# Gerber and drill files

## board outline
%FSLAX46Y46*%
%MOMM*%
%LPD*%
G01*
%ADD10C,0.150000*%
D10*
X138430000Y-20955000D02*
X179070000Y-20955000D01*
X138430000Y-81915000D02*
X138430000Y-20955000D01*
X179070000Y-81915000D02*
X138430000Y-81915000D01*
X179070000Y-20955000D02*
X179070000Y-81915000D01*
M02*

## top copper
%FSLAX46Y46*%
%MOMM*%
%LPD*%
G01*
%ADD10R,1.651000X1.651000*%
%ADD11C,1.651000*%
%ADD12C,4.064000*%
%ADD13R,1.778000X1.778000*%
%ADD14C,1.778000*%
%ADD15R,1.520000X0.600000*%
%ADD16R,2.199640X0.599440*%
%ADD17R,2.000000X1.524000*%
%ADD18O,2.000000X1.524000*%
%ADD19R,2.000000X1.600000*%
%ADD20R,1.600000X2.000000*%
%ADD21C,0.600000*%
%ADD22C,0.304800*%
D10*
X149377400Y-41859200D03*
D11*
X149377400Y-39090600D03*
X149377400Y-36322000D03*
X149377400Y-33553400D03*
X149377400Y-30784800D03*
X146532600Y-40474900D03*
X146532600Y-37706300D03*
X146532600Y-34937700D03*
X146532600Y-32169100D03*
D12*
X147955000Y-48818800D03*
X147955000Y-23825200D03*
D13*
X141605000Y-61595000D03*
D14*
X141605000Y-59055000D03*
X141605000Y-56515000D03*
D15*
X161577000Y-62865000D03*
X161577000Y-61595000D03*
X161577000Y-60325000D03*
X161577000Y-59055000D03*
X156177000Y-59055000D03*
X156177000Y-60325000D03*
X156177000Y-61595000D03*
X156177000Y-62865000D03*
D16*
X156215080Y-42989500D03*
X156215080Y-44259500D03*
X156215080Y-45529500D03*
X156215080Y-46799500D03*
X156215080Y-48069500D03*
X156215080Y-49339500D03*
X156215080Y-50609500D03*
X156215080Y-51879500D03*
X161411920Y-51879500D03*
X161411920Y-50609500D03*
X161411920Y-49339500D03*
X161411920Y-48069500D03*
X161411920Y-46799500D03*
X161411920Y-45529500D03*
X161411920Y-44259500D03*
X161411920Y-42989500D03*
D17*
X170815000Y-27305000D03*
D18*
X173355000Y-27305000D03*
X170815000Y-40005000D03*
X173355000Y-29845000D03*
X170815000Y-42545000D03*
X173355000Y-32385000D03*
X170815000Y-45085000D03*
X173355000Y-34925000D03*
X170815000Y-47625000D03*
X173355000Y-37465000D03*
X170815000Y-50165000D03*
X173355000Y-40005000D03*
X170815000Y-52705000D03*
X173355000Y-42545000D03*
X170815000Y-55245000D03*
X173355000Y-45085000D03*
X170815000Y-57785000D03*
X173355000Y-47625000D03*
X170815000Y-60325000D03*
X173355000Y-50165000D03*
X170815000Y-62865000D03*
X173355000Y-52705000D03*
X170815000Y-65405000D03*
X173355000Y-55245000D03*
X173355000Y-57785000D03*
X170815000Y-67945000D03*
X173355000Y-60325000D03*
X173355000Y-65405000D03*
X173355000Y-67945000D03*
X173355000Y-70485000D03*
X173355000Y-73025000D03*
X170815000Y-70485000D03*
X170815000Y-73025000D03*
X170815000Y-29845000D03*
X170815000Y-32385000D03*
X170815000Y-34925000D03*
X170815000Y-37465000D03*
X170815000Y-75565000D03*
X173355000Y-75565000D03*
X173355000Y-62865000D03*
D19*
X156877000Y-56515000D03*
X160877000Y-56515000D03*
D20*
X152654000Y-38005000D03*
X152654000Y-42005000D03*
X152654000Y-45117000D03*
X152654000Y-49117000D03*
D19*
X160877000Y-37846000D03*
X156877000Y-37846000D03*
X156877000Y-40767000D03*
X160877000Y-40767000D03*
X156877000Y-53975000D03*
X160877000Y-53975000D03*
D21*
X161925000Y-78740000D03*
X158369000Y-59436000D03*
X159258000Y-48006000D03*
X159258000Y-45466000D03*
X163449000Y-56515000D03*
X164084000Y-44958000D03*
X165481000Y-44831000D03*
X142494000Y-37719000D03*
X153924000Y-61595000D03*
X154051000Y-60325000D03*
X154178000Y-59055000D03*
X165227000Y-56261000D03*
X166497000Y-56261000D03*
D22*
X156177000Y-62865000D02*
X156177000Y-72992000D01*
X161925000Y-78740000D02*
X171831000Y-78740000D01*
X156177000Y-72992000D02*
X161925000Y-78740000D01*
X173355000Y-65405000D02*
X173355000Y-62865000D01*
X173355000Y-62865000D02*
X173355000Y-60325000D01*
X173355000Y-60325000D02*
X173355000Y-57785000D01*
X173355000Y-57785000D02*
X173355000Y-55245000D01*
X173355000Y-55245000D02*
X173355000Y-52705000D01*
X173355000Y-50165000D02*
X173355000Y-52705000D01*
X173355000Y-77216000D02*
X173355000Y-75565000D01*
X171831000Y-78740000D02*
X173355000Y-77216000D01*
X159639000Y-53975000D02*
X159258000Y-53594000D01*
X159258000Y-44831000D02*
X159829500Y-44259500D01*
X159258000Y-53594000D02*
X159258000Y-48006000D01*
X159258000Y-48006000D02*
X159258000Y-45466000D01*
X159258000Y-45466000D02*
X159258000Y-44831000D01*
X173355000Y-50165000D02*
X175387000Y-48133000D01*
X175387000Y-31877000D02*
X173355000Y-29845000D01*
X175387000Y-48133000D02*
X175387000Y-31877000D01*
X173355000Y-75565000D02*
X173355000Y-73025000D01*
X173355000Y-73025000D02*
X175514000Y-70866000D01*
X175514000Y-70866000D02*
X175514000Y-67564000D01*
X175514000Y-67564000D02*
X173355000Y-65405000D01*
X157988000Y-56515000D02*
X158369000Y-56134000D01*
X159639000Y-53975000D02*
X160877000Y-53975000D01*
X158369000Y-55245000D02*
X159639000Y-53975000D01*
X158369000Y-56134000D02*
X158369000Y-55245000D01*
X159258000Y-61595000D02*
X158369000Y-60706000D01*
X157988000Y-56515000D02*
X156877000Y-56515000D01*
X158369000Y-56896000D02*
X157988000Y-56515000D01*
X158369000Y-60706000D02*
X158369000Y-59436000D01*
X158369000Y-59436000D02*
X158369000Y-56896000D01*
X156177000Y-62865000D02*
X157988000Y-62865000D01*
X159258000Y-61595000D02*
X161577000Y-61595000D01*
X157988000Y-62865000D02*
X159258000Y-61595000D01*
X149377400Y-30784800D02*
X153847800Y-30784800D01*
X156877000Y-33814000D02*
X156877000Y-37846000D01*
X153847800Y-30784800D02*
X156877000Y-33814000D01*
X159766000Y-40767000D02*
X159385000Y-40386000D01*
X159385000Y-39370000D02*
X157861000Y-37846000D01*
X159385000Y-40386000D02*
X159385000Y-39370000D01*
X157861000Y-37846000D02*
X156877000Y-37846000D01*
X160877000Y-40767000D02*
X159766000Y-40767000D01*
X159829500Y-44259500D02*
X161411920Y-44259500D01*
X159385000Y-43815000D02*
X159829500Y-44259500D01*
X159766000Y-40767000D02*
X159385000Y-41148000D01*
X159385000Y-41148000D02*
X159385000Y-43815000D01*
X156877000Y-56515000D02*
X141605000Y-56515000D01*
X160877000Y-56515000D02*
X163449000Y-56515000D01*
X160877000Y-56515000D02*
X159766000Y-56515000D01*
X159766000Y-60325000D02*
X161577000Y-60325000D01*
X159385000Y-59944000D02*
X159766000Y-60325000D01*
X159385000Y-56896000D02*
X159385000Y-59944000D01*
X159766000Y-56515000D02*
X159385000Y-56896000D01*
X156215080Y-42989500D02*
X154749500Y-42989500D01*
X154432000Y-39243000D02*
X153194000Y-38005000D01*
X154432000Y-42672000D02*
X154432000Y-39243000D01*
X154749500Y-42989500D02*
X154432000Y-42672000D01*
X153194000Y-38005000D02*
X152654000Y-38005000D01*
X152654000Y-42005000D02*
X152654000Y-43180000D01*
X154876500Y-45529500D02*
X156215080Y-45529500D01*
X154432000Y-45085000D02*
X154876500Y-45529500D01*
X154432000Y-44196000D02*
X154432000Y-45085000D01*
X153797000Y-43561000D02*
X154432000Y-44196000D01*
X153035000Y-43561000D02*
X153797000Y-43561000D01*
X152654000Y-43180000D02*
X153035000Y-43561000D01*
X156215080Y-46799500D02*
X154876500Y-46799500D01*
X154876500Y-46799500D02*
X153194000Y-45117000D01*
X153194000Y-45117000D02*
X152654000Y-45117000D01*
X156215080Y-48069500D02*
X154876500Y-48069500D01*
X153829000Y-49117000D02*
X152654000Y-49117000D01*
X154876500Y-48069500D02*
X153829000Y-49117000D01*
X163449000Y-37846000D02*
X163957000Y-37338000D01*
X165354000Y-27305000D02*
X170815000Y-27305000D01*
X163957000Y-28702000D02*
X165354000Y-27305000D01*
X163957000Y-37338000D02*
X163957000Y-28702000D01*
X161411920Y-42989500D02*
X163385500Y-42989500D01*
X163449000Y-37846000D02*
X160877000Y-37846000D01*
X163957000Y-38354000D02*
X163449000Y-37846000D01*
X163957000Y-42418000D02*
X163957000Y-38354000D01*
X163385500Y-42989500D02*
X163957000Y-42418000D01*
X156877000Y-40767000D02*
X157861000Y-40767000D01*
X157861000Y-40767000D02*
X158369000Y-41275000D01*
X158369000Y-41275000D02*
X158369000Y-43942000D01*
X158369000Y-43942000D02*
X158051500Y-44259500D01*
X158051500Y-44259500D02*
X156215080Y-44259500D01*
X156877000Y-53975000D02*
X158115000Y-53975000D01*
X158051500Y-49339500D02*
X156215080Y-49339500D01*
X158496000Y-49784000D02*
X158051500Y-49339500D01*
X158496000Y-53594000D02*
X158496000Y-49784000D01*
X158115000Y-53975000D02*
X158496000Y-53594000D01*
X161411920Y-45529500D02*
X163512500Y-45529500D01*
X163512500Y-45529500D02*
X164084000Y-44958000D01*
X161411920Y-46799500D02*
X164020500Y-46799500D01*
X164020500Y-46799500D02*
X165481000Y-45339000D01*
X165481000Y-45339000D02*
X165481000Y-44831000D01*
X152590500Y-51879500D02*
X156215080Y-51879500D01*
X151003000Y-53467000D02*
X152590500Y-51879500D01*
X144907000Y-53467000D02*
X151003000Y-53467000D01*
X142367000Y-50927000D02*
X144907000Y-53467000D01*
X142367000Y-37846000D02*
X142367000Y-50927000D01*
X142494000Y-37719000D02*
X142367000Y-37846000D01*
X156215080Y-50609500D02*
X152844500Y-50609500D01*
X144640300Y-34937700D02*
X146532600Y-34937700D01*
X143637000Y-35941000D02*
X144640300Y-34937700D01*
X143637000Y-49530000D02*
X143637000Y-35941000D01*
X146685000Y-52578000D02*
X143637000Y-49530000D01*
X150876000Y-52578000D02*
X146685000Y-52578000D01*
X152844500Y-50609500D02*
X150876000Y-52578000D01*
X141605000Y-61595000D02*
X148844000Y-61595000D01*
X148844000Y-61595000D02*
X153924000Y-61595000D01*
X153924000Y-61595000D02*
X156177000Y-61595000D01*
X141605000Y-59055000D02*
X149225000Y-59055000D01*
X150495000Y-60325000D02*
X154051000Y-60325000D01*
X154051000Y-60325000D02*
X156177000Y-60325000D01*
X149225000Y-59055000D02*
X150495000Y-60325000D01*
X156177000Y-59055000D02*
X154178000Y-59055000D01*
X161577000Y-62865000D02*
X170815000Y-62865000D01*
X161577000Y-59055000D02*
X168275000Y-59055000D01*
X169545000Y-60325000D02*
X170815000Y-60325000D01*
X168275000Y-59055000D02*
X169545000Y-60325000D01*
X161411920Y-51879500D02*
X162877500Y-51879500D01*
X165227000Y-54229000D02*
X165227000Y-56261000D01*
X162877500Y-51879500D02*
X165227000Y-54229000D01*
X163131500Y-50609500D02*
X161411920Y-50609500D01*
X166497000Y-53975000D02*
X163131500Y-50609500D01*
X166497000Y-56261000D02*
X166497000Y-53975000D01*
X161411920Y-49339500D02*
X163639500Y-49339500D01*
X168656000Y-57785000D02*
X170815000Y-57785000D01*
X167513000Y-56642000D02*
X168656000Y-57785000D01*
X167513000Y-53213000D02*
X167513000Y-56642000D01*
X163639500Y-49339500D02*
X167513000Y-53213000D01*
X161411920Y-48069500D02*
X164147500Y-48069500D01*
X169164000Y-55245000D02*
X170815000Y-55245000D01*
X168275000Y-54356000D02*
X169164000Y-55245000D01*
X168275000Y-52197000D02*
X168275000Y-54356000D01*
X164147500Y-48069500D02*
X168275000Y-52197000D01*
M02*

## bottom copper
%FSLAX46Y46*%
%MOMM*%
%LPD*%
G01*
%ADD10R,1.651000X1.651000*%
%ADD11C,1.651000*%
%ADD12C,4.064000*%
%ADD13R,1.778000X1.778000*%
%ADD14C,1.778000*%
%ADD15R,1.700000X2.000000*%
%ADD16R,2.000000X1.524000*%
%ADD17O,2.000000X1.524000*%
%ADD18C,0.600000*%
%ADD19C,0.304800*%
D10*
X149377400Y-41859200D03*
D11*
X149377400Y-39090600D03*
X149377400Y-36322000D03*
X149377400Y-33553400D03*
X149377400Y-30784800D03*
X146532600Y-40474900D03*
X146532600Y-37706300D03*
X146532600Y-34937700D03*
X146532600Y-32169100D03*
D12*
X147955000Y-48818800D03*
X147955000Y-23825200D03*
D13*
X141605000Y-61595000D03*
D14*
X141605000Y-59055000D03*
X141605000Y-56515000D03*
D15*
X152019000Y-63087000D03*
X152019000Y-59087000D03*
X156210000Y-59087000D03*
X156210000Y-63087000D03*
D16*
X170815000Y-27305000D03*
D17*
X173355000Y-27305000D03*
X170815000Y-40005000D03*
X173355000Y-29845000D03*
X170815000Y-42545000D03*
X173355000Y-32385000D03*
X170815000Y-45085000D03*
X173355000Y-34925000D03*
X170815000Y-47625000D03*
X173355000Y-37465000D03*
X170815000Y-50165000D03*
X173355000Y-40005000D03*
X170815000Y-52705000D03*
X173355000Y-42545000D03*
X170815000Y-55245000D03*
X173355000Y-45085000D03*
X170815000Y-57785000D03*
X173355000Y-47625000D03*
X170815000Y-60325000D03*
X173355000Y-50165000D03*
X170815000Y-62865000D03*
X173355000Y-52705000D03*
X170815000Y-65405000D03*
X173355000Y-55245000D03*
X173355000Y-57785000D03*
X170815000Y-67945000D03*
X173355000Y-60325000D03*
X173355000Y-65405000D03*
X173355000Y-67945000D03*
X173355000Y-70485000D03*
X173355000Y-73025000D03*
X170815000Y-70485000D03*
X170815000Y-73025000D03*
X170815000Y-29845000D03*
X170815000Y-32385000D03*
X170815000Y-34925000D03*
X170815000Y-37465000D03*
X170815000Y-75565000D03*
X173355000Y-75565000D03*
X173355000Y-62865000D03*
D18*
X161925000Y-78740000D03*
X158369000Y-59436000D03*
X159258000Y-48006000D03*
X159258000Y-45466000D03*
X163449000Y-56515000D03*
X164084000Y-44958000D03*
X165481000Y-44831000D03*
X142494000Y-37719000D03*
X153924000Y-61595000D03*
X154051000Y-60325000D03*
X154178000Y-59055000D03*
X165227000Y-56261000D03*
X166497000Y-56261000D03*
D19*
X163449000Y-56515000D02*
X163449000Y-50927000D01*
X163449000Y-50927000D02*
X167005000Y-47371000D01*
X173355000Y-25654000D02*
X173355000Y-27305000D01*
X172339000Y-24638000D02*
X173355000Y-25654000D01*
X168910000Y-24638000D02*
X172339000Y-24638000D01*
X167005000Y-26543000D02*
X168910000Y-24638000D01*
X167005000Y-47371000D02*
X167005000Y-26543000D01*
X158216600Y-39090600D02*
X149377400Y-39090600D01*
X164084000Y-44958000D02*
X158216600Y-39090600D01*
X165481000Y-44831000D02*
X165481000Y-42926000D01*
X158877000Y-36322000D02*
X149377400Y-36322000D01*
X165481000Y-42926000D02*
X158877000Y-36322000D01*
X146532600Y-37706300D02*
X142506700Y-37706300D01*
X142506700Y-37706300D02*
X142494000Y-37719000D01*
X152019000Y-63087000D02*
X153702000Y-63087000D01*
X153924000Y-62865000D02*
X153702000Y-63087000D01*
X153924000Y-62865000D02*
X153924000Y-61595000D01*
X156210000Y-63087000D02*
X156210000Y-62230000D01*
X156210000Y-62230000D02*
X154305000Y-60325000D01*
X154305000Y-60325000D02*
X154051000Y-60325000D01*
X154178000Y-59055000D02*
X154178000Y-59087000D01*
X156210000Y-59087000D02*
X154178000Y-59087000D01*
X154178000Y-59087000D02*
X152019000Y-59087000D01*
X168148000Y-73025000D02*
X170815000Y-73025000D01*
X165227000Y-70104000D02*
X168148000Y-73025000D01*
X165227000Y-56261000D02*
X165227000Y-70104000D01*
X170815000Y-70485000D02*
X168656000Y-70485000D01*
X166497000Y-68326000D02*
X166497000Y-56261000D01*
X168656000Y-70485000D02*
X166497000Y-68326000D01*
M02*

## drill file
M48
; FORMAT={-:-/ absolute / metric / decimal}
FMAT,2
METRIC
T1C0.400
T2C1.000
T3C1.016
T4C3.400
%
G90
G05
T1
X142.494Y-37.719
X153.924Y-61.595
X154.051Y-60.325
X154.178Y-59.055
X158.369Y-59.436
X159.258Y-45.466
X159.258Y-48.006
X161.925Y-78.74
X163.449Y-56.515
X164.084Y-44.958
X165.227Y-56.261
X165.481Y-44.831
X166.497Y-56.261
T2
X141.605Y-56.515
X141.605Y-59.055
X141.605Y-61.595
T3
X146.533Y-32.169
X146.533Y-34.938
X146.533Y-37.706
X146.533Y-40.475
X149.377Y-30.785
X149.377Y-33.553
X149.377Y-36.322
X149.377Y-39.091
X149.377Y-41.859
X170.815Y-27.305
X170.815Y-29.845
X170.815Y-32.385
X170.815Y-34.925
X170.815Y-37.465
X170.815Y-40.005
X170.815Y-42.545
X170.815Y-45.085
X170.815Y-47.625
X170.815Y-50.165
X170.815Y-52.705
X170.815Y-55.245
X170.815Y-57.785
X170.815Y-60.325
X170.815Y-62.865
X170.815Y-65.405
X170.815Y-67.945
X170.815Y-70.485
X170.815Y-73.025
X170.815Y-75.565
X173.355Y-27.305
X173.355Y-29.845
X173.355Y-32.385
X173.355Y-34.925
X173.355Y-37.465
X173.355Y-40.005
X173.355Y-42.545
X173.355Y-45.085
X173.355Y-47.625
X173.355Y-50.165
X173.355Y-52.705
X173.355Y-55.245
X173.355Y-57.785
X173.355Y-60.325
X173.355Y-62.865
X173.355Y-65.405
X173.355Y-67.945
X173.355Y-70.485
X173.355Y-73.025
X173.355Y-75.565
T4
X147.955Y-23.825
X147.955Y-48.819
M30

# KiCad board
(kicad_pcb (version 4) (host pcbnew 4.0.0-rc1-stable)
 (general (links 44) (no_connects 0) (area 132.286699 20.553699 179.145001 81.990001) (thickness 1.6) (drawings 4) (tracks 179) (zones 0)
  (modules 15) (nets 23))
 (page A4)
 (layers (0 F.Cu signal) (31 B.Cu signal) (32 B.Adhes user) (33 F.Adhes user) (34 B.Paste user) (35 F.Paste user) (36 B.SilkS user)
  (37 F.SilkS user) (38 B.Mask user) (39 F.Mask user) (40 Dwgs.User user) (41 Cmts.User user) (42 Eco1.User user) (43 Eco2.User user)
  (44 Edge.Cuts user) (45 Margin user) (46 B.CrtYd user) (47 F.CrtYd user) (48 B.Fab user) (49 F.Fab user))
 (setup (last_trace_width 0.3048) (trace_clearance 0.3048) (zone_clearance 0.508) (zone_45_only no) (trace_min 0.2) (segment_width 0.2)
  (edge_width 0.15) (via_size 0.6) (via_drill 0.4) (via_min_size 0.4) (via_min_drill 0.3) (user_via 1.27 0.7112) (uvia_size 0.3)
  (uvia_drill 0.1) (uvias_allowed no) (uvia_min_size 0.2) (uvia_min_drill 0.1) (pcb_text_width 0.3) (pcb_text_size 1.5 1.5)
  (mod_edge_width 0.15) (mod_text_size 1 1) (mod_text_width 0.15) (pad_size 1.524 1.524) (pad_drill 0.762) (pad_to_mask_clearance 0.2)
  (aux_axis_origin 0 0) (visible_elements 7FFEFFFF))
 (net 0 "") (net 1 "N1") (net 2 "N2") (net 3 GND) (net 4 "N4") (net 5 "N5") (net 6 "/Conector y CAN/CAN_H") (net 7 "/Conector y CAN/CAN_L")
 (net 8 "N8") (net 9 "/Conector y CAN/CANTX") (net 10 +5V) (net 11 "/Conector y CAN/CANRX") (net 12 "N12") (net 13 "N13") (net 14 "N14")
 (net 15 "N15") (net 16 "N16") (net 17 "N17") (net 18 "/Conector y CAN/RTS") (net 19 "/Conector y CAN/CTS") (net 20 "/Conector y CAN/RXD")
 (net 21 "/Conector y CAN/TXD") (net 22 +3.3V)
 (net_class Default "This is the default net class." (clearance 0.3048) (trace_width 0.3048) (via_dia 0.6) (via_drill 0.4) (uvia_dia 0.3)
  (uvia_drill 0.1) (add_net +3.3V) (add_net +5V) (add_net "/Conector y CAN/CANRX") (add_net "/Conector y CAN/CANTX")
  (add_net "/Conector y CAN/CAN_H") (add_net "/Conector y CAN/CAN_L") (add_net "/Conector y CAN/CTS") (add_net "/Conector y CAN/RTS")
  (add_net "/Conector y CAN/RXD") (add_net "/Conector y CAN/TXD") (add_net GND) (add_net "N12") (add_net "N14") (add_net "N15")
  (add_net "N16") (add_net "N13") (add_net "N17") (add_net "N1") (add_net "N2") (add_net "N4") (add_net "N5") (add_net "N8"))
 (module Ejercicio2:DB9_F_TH (layer F.Cu) (at 147.955 36.322 90)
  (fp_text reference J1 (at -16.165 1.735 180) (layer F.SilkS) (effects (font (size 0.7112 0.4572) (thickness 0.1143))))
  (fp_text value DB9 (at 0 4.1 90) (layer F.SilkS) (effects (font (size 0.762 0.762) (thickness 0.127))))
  (pad 1 thru_hole rect (at -5.5372 1.4224 90) (size 1.651 1.651) (drill 1.016) (layers *.Cu *.Mask))
  (pad 2 thru_hole circle (at -2.7686 1.4224 90) (size 1.651 1.651) (drill 1.016) (layers *.Cu *.Mask) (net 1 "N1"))
  (pad 3 thru_hole circle (at 0 1.4224 90) (size 1.651 1.651) (drill 1.016) (layers *.Cu *.Mask) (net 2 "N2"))
  (pad 4 thru_hole circle (at 2.7686 1.4224 90) (size 1.651 1.651) (drill 1.016) (layers *.Cu *.Mask))
  (pad 5 thru_hole circle (at 5.5372 1.4224 90) (size 1.651 1.651) (drill 1.016) (layers *.Cu *.Mask) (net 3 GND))
  (pad 6 thru_hole circle (at -4.1529 -1.4224 90) (size 1.651 1.651) (drill 1.016) (layers *.Cu *.Mask))
  (pad 7 thru_hole circle (at -1.3843 -1.4224 90) (size 1.651 1.651) (drill 1.016) (layers *.Cu *.Mask) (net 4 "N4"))
  (pad 8 thru_hole circle (at 1.3843 -1.4224 90) (size 1.651 1.651) (drill 1.016) (layers *.Cu *.Mask) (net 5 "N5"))
  (pad 9 thru_hole circle (at 4.1529 -1.4224 90) (size 1.651 1.651) (drill 1.016) (layers *.Cu *.Mask))
  (pad 10 thru_hole circle (at -12.4968 0 90) (size 4.064 4.064) (drill 3.4) (layers *.Cu *.Mask))
  (pad 11 thru_hole circle (at 12.4968 0 90) (size 4.064 4.064) (drill 3.4) (layers *.Cu *.Mask)))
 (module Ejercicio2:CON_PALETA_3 (layer F.Cu) (at 141.605 59.055 90)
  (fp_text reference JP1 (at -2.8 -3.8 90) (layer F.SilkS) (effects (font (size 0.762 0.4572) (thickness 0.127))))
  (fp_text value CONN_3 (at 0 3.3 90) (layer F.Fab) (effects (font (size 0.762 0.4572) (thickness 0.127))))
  (pad 1 thru_hole rect (at -2.54 0 90) (size 1.778 1.778) (drill 1) (layers *.Cu *.Mask) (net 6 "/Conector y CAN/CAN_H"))
  (pad 2 thru_hole circle (at 0 0 90) (size 1.778 1.778) (drill 1) (layers *.Cu *.Mask) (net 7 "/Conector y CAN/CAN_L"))
  (pad 3 thru_hole circle (at 2.54 0 90) (size 1.778 1.778) (drill 1) (layers *.Cu *.Mask) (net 3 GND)))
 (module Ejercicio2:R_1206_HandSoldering (layer B.Cu) (at 152.019 61.087 90)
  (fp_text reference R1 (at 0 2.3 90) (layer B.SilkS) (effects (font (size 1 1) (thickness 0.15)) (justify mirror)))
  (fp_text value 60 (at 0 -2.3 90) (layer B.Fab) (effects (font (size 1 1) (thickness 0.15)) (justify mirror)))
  (pad 1 smd rect (at -2 0 90) (size 2 1.7) (layers B.Cu B.Paste B.Mask) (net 6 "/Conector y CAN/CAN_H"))
  (pad 2 smd rect (at 2 0 90) (size 2 1.7) (layers B.Cu B.Paste B.Mask) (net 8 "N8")))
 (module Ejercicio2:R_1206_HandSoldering (layer B.Cu) (at 156.21 61.087 270)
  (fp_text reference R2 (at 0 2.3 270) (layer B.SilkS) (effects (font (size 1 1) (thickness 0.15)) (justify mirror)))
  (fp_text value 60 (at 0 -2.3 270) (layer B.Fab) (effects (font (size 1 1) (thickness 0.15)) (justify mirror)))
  (pad 1 smd rect (at -2 0 270) (size 2 1.7) (layers B.Cu B.Paste B.Mask) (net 8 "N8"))
  (pad 2 smd rect (at 2 0 270) (size 2 1.7) (layers B.Cu B.Paste B.Mask) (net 7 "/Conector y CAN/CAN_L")))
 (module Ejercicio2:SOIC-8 (layer F.Cu) (at 158.877 60.96 180)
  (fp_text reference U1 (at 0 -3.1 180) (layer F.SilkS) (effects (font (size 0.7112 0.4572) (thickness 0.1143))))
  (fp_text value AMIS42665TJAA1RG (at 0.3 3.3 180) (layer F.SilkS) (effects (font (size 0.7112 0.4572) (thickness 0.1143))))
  (pad 1 smd rect (at -2.7 -1.905 90) (size 0.6 1.52) (layers F.Cu F.Paste F.Mask) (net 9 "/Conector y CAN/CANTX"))
  (pad 2 smd rect (at -2.7 -0.635 90) (size 0.6 1.52) (layers F.Cu F.Paste F.Mask) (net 3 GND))
  (pad 3 smd rect (at -2.7 0.635 90) (size 0.6 1.52) (layers F.Cu F.Paste F.Mask) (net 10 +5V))
  (pad 4 smd rect (at -2.7 1.905 90) (size 0.6 1.52) (layers F.Cu F.Paste F.Mask) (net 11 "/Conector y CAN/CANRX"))
  (pad 5 smd rect (at 2.7 1.905 90) (size 0.6 1.52) (layers F.Cu F.Paste F.Mask) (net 8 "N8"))
  (pad 6 smd rect (at 2.7 0.635 90) (size 0.6 1.52) (layers F.Cu F.Paste F.Mask) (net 7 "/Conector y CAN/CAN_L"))
  (pad 7 smd rect (at 2.7 -0.635 90) (size 0.6 1.52) (layers F.Cu F.Paste F.Mask) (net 6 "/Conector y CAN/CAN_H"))
  (pad 8 smd rect (at 2.7 -1.905 90) (size 0.6 1.52) (layers F.Cu F.Paste F.Mask) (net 3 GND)))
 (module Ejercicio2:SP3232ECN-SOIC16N (layer F.Cu) (at 158.8135 47.4345 270)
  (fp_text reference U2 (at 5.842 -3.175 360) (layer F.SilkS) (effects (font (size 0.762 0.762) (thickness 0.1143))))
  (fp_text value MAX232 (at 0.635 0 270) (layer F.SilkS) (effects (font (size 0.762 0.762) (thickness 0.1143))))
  (pad 1 smd rect (at -4.445 2.59842 270) (size 0.59944 2.19964) (layers F.Cu F.Paste F.Mask) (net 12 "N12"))
  (pad 2 smd rect (at -3.175 2.59842 270) (size 0.59944 2.19964) (layers F.Cu F.Paste F.Mask) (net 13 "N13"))
  (pad 3 smd rect (at -1.905 2.59842 270) (size 0.59944 2.19964) (layers F.Cu F.Paste F.Mask) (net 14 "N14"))
  (pad 4 smd rect (at -0.635 2.59842 270) (size 0.59944 2.19964) (layers F.Cu F.Paste F.Mask) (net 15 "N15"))
  (pad 5 smd rect (at 0.635 2.59842 270) (size 0.59944 2.19964) (layers F.Cu F.Paste F.Mask) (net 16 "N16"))
  (pad 6 smd rect (at 1.905 2.59842 270) (size 0.59944 2.19964) (layers F.Cu F.Paste F.Mask) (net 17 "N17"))
  (pad 7 smd rect (at 3.175 2.59842 270) (size 0.59944 2.19964) (layers F.Cu F.Paste F.Mask) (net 5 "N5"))
  (pad 8 smd rect (at 4.445 2.59842 270) (size 0.59944 2.19964) (layers F.Cu F.Paste F.Mask) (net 4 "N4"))
  (pad 9 smd rect (at 4.445 -2.59842 270) (size 0.59944 2.19964) (layers F.Cu F.Paste F.Mask) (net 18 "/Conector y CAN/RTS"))
  (pad 10 smd rect (at 3.175 -2.59842 270) (size 0.59944 2.19964) (layers F.Cu F.Paste F.Mask) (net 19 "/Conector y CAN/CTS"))
  (pad 11 smd rect (at 1.905 -2.59842 270) (size 0.59944 2.19964) (layers F.Cu F.Paste F.Mask) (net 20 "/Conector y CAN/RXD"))
  (pad 12 smd rect (at 0.635 -2.59842 270) (size 0.59944 2.19964) (layers F.Cu F.Paste F.Mask) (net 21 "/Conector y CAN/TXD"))
  (pad 13 smd rect (at -0.635 -2.59842 270) (size 0.59944 2.19964) (layers F.Cu F.Paste F.Mask) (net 2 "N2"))
  (pad 14 smd rect (at -1.905 -2.59842 270) (size 0.59944 2.19964) (layers F.Cu F.Paste F.Mask) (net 1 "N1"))
  (pad 15 smd rect (at -3.175 -2.59842 270) (size 0.59944 2.19964) (layers F.Cu F.Paste F.Mask) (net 3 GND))
  (pad 16 smd rect (at -4.445 -2.59842 270) (size 0.59944 2.19964) (layers F.Cu F.Paste F.Mask) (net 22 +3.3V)))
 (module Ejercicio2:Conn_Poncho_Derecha (layer F.Cu) (at 170.815 27.305)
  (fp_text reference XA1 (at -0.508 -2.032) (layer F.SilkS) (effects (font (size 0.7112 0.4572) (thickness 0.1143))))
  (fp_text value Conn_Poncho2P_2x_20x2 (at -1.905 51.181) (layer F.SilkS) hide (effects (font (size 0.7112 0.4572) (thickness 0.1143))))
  (pad 1 thru_hole rect (at 0 0 270) (size 1.524 2) (drill 1.016) (layers *.Cu *.Mask) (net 22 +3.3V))
  (pad 2 thru_hole oval (at 2.54 0 270) (size 1.524 2) (drill 1.016) (layers *.Cu *.Mask) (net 10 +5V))
  (pad 11 thru_hole oval (at 0 12.7 270) (size 1.524 2) (drill 1.016) (layers *.Cu *.Mask))
  (pad 4 thru_hole oval (at 2.54 2.54 270) (size 1.524 2) (drill 1.016) (layers *.Cu *.Mask) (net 3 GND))
  (pad 13 thru_hole oval (at 0 15.24 270) (size 1.524 2) (drill 1.016) (layers *.Cu *.Mask))
  (pad 6 thru_hole oval (at 2.54 5.08 270) (size 1.524 2) (drill 1.016) (layers *.Cu *.Mask))
  (pad 15 thru_hole oval (at 0 17.78 270) (size 1.524 2) (drill 1.016) (layers *.Cu *.Mask))
  (pad 8 thru_hole oval (at 2.54 7.62 270) (size 1.524 2) (drill 1.016) (layers *.Cu *.Mask))
  (pad 17 thru_hole oval (at 0 20.32 270) (size 1.524 2) (drill 1.016) (layers *.Cu *.Mask))
  (pad 10 thru_hole oval (at 2.54 10.16 270) (size 1.524 2) (drill 1.016) (layers *.Cu *.Mask))
  (pad 19 thru_hole oval (at 0 22.86 270) (size 1.524 2) (drill 1.016) (layers *.Cu *.Mask))
  (pad 12 thru_hole oval (at 2.54 12.7 270) (size 1.524 2) (drill 1.016) (layers *.Cu *.Mask))
  (pad 21 thru_hole oval (at 0 25.4 270) (size 1.524 2) (drill 1.016) (layers *.Cu *.Mask))
  (pad 14 thru_hole oval (at 2.54 15.24 270) (size 1.524 2) (drill 1.016) (layers *.Cu *.Mask))
  (pad 23 thru_hole oval (at 0 27.94 270) (size 1.524 2) (drill 1.016) (layers *.Cu *.Mask) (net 21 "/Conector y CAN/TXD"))
  (pad 16 thru_hole oval (at 2.54 17.78 270) (size 1.524 2) (drill 1.016) (layers *.Cu *.Mask))
  (pad 25 thru_hole oval (at 0 30.48 270) (size 1.524 2) (drill 1.016) (layers *.Cu *.Mask) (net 20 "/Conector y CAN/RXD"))
  (pad 18 thru_hole oval (at 2.54 20.32 270) (size 1.524 2) (drill 1.016) (layers *.Cu *.Mask))
  (pad 27 thru_hole oval (at 0 33.02 270) (size 1.524 2) (drill 1.016) (layers *.Cu *.Mask) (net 11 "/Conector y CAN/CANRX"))
  (pad 20 thru_hole oval (at 2.54 22.86 270) (size 1.524 2) (drill 1.016) (layers *.Cu *.Mask) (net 3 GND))
  (pad 29 thru_hole oval (at 0 35.56 270) (size 1.524 2) (drill 1.016) (layers *.Cu *.Mask) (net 9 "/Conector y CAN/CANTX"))
  (pad 22 thru_hole oval (at 2.54 25.4 270) (size 1.524 2) (drill 1.016) (layers *.Cu *.Mask) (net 3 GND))
  (pad 31 thru_hole oval (at 0 38.1 270) (size 1.524 2) (drill 1.016) (layers *.Cu *.Mask))
  (pad 24 thru_hole oval (at 2.54 27.94 270) (size 1.524 2) (drill 1.016) (layers *.Cu *.Mask) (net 3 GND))
  (pad 26 thru_hole oval (at 2.54 30.48 270) (size 1.524 2) (drill 1.016) (layers *.Cu *.Mask) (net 3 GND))
  (pad 33 thru_hole oval (at 0 40.64 270) (size 1.524 2) (drill 1.016) (layers *.Cu *.Mask))
  (pad 28 thru_hole oval (at 2.54 33.02 270) (size 1.524 2) (drill 1.016) (layers *.Cu *.Mask) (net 3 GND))
  (pad 32 thru_hole oval (at 2.54 38.1 270) (size 1.524 2) (drill 1.016) (layers *.Cu *.Mask) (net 3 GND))
  (pad 34 thru_hole oval (at 2.54 40.64 270) (size 1.524 2) (drill 1.016) (layers *.Cu *.Mask))
  (pad 36 thru_hole oval (at 2.54 43.18 270) (size 1.524 2) (drill 1.016) (layers *.Cu *.Mask))
  (pad 38 thru_hole oval (at 2.54 45.72 270) (size 1.524 2) (drill 1.016) (layers *.Cu *.Mask) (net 3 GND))
  (pad 35 thru_hole oval (at 0 43.18 270) (size 1.524 2) (drill 1.016) (layers *.Cu *.Mask) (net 19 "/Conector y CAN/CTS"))
  (pad 37 thru_hole oval (at 0 45.72 270) (size 1.524 2) (drill 1.016) (layers *.Cu *.Mask) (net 18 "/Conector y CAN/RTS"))
  (pad 3 thru_hole oval (at 0 2.54 270) (size 1.524 2) (drill 1.016) (layers *.Cu *.Mask))
  (pad 5 thru_hole oval (at 0 5.08 270) (size 1.524 2) (drill 1.016) (layers *.Cu *.Mask))
  (pad 7 thru_hole oval (at 0 7.62 270) (size 1.524 2) (drill 1.016) (layers *.Cu *.Mask))
  (pad 9 thru_hole oval (at 0 10.16 270) (size 1.524 2) (drill 1.016) (layers *.Cu *.Mask))
  (pad 39 thru_hole oval (at 0 48.26 270) (size 1.524 2) (drill 1.016) (layers *.Cu *.Mask))
  (pad 40 thru_hole oval (at 2.54 48.26 270) (size 1.524 2) (drill 1.016) (layers *.Cu *.Mask) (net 3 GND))
  (pad 30 thru_hole oval (at 2.54 35.56 270) (size 1.524 2) (drill 1.016) (layers *.Cu *.Mask) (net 3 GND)))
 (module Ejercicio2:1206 (layer F.Cu) (at 158.877 56.515)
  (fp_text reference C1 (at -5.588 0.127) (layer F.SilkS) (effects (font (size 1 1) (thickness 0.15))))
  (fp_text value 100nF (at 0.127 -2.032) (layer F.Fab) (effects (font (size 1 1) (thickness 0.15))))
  (pad 1 smd rect (at -2 0) (size 2 1.6) (layers F.Cu F.Paste F.Mask) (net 3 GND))
  (pad 2 smd rect (at 2 0) (size 2 1.6) (layers F.Cu F.Paste F.Mask) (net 10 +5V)))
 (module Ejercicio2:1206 (layer F.Cu) (at 152.654 40.005 270)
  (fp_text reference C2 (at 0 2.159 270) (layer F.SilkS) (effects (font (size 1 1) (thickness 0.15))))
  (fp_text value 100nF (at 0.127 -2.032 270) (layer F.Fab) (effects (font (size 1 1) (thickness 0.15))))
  (pad 1 smd rect (at -2 0 270) (size 2 1.6) (layers F.Cu F.Paste F.Mask) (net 12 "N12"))
  (pad 2 smd rect (at 2 0 270) (size 2 1.6) (layers F.Cu F.Paste F.Mask) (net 14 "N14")))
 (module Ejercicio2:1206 (layer F.Cu) (at 152.654 47.117 270)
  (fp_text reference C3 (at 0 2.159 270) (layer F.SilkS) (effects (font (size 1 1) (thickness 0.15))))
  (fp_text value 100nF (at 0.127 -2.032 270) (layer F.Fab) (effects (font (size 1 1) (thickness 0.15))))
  (pad 1 smd rect (at -2 0 270) (size 2 1.6) (layers F.Cu F.Paste F.Mask) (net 15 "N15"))
  (pad 2 smd rect (at 2 0 270) (size 2 1.6) (layers F.Cu F.Paste F.Mask) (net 16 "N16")))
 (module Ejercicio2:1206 (layer F.Cu) (at 158.877 37.846 180)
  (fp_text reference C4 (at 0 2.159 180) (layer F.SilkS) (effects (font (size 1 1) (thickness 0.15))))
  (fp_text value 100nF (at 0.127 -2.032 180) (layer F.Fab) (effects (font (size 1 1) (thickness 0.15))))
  (pad 1 smd rect (at -2 0 180) (size 2 1.6) (layers F.Cu F.Paste F.Mask) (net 22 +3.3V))
  (pad 2 smd rect (at 2 0 180) (size 2 1.6) (layers F.Cu F.Paste F.Mask) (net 3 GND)))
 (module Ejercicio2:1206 (layer F.Cu) (at 158.877 40.767)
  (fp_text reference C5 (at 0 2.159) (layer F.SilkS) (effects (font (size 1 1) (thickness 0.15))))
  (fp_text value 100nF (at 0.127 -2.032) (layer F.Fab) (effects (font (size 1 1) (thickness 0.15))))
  (pad 1 smd rect (at -2 0) (size 2 1.6) (layers F.Cu F.Paste F.Mask) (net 13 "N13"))
  (pad 2 smd rect (at 2 0) (size 2 1.6) (layers F.Cu F.Paste F.Mask) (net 3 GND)))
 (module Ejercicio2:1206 (layer F.Cu) (at 158.877 53.975)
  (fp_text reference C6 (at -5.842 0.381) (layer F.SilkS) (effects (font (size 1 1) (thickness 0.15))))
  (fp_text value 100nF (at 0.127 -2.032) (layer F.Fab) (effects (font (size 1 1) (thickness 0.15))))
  (pad 1 smd rect (at -2 0) (size 2 1.6) (layers F.Cu F.Paste F.Mask) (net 17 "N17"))
  (pad 2 smd rect (at 2 0) (size 2 1.6) (layers F.Cu F.Paste F.Mask) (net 3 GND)))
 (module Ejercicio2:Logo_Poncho (layer F.Cu) (at 158.877 73.787)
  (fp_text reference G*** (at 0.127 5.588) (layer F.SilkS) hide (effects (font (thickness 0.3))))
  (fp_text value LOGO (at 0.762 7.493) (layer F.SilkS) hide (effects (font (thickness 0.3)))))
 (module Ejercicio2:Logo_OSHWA (layer F.Cu) (at 158.877 27.178)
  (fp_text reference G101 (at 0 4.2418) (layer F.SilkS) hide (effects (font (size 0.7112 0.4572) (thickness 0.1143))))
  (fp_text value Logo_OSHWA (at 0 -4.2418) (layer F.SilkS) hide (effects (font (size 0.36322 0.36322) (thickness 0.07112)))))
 (gr_line (start 138.43 20.955) (end 179.07 20.955) (angle 90) (layer Edge.Cuts) (width 0.15))
 (gr_line (start 138.43 81.915) (end 138.43 20.955) (angle 90) (layer Edge.Cuts) (width 0.15))
 (gr_line (start 179.07 81.915) (end 138.43 81.915) (angle 90) (layer Edge.Cuts) (width 0.15))
 (gr_line (start 179.07 20.955) (end 179.07 81.915) (angle 90) (layer Edge.Cuts) (width 0.15))
 (via (at 161.925 78.74) (size 0.6) (drill 0.4) (layers F.Cu B.Cu) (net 3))
 (segment (start 156.177 62.865) (end 156.177 72.992) (width 0.3048) (layer F.Cu) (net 3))
 (segment (start 161.925 78.74) (end 171.831 78.74) (width 0.3048) (layer F.Cu) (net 3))
 (segment (start 156.177 72.992) (end 161.925 78.74) (width 0.3048) (layer F.Cu) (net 3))
 (via (at 158.369 59.436) (size 0.6) (drill 0.4) (layers F.Cu B.Cu) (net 3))
 (via (at 159.258 48.006) (size 0.6) (drill 0.4) (layers F.Cu B.Cu) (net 3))
 (via (at 159.258 45.466) (size 0.6) (drill 0.4) (layers F.Cu B.Cu) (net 3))
 (segment (start 173.355 65.405) (end 173.355 62.865) (width 0.3048) (layer F.Cu) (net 3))
 (segment (start 173.355 62.865) (end 173.355 60.325) (width 0.3048) (layer F.Cu) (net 3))
 (segment (start 173.355 60.325) (end 173.355 57.785) (width 0.3048) (layer F.Cu) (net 3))
 (segment (start 173.355 57.785) (end 173.355 55.245) (width 0.3048) (layer F.Cu) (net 3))
 (segment (start 173.355 55.245) (end 173.355 52.705) (width 0.3048) (layer F.Cu) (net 3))
 (segment (start 173.355 50.165) (end 173.355 52.705) (width 0.3048) (layer F.Cu) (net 3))
 (segment (start 173.355 77.216) (end 173.355 75.565) (width 0.3048) (layer F.Cu) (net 3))
 (segment (start 171.831 78.74) (end 173.355 77.216) (width 0.3048) (layer F.Cu) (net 3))
 (segment (start 159.639 53.975) (end 159.258 53.594) (width 0.3048) (layer F.Cu) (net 3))
 (segment (start 159.258 44.831) (end 159.8295 44.2595) (width 0.3048) (layer F.Cu) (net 3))
 (segment (start 159.258 53.594) (end 159.258 48.006) (width 0.3048) (layer F.Cu) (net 3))
 (segment (start 159.258 48.006) (end 159.258 45.466) (width 0.3048) (layer F.Cu) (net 3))
 (segment (start 159.258 45.466) (end 159.258 44.831) (width 0.3048) (layer F.Cu) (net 3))
 (segment (start 173.355 50.165) (end 175.387 48.133) (width 0.3048) (layer F.Cu) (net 3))
 (segment (start 175.387 31.877) (end 173.355 29.845) (width 0.3048) (layer F.Cu) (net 3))
 (segment (start 175.387 48.133) (end 175.387 31.877) (width 0.3048) (layer F.Cu) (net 3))
 (segment (start 173.355 75.565) (end 173.355 73.025) (width 0.3048) (layer F.Cu) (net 3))
 (segment (start 173.355 73.025) (end 175.514 70.866) (width 0.3048) (layer F.Cu) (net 3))
 (segment (start 175.514 70.866) (end 175.514 67.564) (width 0.3048) (layer F.Cu) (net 3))
 (segment (start 175.514 67.564) (end 173.355 65.405) (width 0.3048) (layer F.Cu) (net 3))
 (segment (start 157.988 56.515) (end 158.369 56.134) (width 0.3048) (layer F.Cu) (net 3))
 (segment (start 159.639 53.975) (end 160.877 53.975) (width 0.3048) (layer F.Cu) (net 3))
 (segment (start 158.369 55.245) (end 159.639 53.975) (width 0.3048) (layer F.Cu) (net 3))
 (segment (start 158.369 56.134) (end 158.369 55.245) (width 0.3048) (layer F.Cu) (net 3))
 (segment (start 159.258 61.595) (end 158.369 60.706) (width 0.3048) (layer F.Cu) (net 3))
 (segment (start 157.988 56.515) (end 156.877 56.515) (width 0.3048) (layer F.Cu) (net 3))
 (segment (start 158.369 56.896) (end 157.988 56.515) (width 0.3048) (layer F.Cu) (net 3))
 (segment (start 158.369 60.706) (end 158.369 59.436) (width 0.3048) (layer F.Cu) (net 3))
 (segment (start 158.369 59.436) (end 158.369 56.896) (width 0.3048) (layer F.Cu) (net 3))
 (segment (start 156.177 62.865) (end 157.988 62.865) (width 0.3048) (layer F.Cu) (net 3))
 (segment (start 159.258 61.595) (end 161.577 61.595) (width 0.3048) (layer F.Cu) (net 3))
 (segment (start 157.988 62.865) (end 159.258 61.595) (width 0.3048) (layer F.Cu) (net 3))
 (segment (start 149.3774 30.7848) (end 153.8478 30.7848) (width 0.3048) (layer F.Cu) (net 3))
 (segment (start 156.877 33.814) (end 156.877 37.846) (width 0.3048) (layer F.Cu) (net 3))
 (segment (start 153.8478 30.7848) (end 156.877 33.814) (width 0.3048) (layer F.Cu) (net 3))
 (segment (start 159.766 40.767) (end 159.385 40.386) (width 0.3048) (layer F.Cu) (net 3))
 (segment (start 159.385 39.37) (end 157.861 37.846) (width 0.3048) (layer F.Cu) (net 3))
 (segment (start 159.385 40.386) (end 159.385 39.37) (width 0.3048) (layer F.Cu) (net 3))
 (segment (start 157.861 37.846) (end 156.877 37.846) (width 0.3048) (layer F.Cu) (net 3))
 (segment (start 160.877 40.767) (end 159.766 40.767) (width 0.3048) (layer F.Cu) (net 3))
 (segment (start 159.8295 44.2595) (end 161.41192 44.2595) (width 0.3048) (layer F.Cu) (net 3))
 (segment (start 159.385 43.815) (end 159.8295 44.2595) (width 0.3048) (layer F.Cu) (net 3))
 (segment (start 159.766 40.767) (end 159.385 41.148) (width 0.3048) (layer F.Cu) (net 3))
 (segment (start 159.385 41.148) (end 159.385 43.815) (width 0.3048) (layer F.Cu) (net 3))
 (segment (start 156.877 56.515) (end 141.605 56.515) (width 0.3048) (layer F.Cu) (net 3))
 (segment (start 163.449 56.515) (end 163.449 50.927) (width 0.3048) (layer B.Cu) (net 10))
 (segment (start 163.449 50.927) (end 167.005 47.371) (width 0.3048) (layer B.Cu) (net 10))
 (segment (start 160.877 56.515) (end 163.449 56.515) (width 0.3048) (layer F.Cu) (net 10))
 (segment (start 173.355 25.654) (end 173.355 27.305) (width 0.3048) (layer B.Cu) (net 10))
 (segment (start 172.339 24.638) (end 173.355 25.654) (width 0.3048) (layer B.Cu) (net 10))
 (segment (start 168.91 24.638) (end 172.339 24.638) (width 0.3048) (layer B.Cu) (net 10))
 (segment (start 167.005 26.543) (end 168.91 24.638) (width 0.3048) (layer B.Cu) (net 10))
 (segment (start 167.005 47.371) (end 167.005 26.543) (width 0.3048) (layer B.Cu) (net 10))
 (via (at 163.449 56.515) (size 0.6) (drill 0.4) (layers F.Cu B.Cu) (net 10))
 (segment (start 160.877 56.515) (end 159.766 56.515) (width 0.3048) (layer F.Cu) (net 10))
 (segment (start 159.766 60.325) (end 161.577 60.325) (width 0.3048) (layer F.Cu) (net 10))
 (segment (start 159.385 59.944) (end 159.766 60.325) (width 0.3048) (layer F.Cu) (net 10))
 (segment (start 159.385 56.896) (end 159.385 59.944) (width 0.3048) (layer F.Cu) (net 10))
 (segment (start 159.766 56.515) (end 159.385 56.896) (width 0.3048) (layer F.Cu) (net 10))
 (segment (start 156.21508 42.9895) (end 154.7495 42.9895) (width 0.3048) (layer F.Cu) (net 12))
 (segment (start 154.432 39.243) (end 153.194 38.005) (width 0.3048) (layer F.Cu) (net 12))
 (segment (start 154.432 42.672) (end 154.432 39.243) (width 0.3048) (layer F.Cu) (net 12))
 (segment (start 154.7495 42.9895) (end 154.432 42.672) (width 0.3048) (layer F.Cu) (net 12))
 (segment (start 153.194 38.005) (end 152.654 38.005) (width 0.3048) (layer F.Cu) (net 12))
 (segment (start 152.654 42.005) (end 152.654 43.18) (width 0.3048) (layer F.Cu) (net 14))
 (segment (start 154.8765 45.5295) (end 156.21508 45.5295) (width 0.3048) (layer F.Cu) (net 14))
 (segment (start 154.432 45.085) (end 154.8765 45.5295) (width 0.3048) (layer F.Cu) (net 14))
 (segment (start 154.432 44.196) (end 154.432 45.085) (width 0.3048) (layer F.Cu) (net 14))
 (segment (start 153.797 43.561) (end 154.432 44.196) (width 0.3048) (layer F.Cu) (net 14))
 (segment (start 153.035 43.561) (end 153.797 43.561) (width 0.3048) (layer F.Cu) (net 14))
 (segment (start 152.654 43.18) (end 153.035 43.561) (width 0.3048) (layer F.Cu) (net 14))
 (segment (start 156.21508 46.7995) (end 154.8765 46.7995) (width 0.3048) (layer F.Cu) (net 15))
 (segment (start 154.8765 46.7995) (end 153.194 45.117) (width 0.3048) (layer F.Cu) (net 15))
 (segment (start 153.194 45.117) (end 152.654 45.117) (width 0.3048) (layer F.Cu) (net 15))
 (segment (start 156.21508 48.0695) (end 154.8765 48.0695) (width 0.3048) (layer F.Cu) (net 16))
 (segment (start 153.829 49.117) (end 152.654 49.117) (width 0.3048) (layer F.Cu) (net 16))
 (segment (start 154.8765 48.0695) (end 153.829 49.117) (width 0.3048) (layer F.Cu) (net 16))
 (segment (start 163.449 37.846) (end 163.957 37.338) (width 0.3048) (layer F.Cu) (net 22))
 (segment (start 165.354 27.305) (end 170.815 27.305) (width 0.3048) (layer F.Cu) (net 22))
 (segment (start 163.957 28.702) (end 165.354 27.305) (width 0.3048) (layer F.Cu) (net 22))
 (segment (start 163.957 37.338) (end 163.957 28.702) (width 0.3048) (layer F.Cu) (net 22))
 (segment (start 161.41192 42.9895) (end 163.3855 42.9895) (width 0.3048) (layer F.Cu) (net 22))
 (segment (start 163.449 37.846) (end 160.877 37.846) (width 0.3048) (layer F.Cu) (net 22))
 (segment (start 163.957 38.354) (end 163.449 37.846) (width 0.3048) (layer F.Cu) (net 22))
 (segment (start 163.957 42.418) (end 163.957 38.354) (width 0.3048) (layer F.Cu) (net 22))
 (segment (start 163.3855 42.9895) (end 163.957 42.418) (width 0.3048) (layer F.Cu) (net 22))
 (segment (start 156.877 40.767) (end 157.861 40.767) (width 0.3048) (layer F.Cu) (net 13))
 (segment (start 157.861 40.767) (end 158.369 41.275) (width 0.3048) (layer F.Cu) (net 13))
 (segment (start 158.369 41.275) (end 158.369 43.942) (width 0.3048) (layer F.Cu) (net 13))
 (segment (start 158.369 43.942) (end 158.0515 44.2595) (width 0.3048) (layer F.Cu) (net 13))
 (segment (start 158.0515 44.2595) (end 156.21508 44.2595) (width 0.3048) (layer F.Cu) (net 13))
 (segment (start 156.877 53.975) (end 158.115 53.975) (width 0.3048) (layer F.Cu) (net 17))
 (segment (start 158.0515 49.3395) (end 156.21508 49.3395) (width 0.3048) (layer F.Cu) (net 17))
 (segment (start 158.496 49.784) (end 158.0515 49.3395) (width 0.3048) (layer F.Cu) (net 17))
 (segment (start 158.496 53.594) (end 158.496 49.784) (width 0.3048) (layer F.Cu) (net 17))
 (segment (start 158.115 53.975) (end 158.496 53.594) (width 0.3048) (layer F.Cu) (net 17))
 (segment (start 161.41192 45.5295) (end 163.5125 45.5295) (width 0.3048) (layer F.Cu) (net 1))
 (segment (start 158.2166 39.0906) (end 149.3774 39.0906) (width 0.3048) (layer B.Cu) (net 1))
 (segment (start 164.084 44.958) (end 158.2166 39.0906) (width 0.3048) (layer B.Cu) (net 1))
 (via (at 164.084 44.958) (size 0.6) (drill 0.4) (layers F.Cu B.Cu) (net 1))
 (segment (start 163.5125 45.5295) (end 164.084 44.958) (width 0.3048) (layer F.Cu) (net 1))
 (segment (start 165.481 44.831) (end 165.481 42.926) (width 0.3048) (layer B.Cu) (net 2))
 (segment (start 158.877 36.322) (end 149.3774 36.322) (width 0.3048) (layer B.Cu) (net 2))
 (segment (start 165.481 42.926) (end 158.877 36.322) (width 0.3048) (layer B.Cu) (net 2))
 (segment (start 161.41192 46.7995) (end 164.0205 46.7995) (width 0.3048) (layer F.Cu) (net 2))
 (segment (start 164.0205 46.7995) (end 165.481 45.339) (width 0.3048) (layer F.Cu) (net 2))
 (segment (start 165.481 45.339) (end 165.481 44.831) (width 0.3048) (layer F.Cu) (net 2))
 (via (at 165.481 44.831) (size 0.6) (drill 0.4) (layers F.Cu B.Cu) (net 2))
 (segment (start 146.5326 37.7063) (end 142.5067 37.7063) (width 0.3048) (layer B.Cu) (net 4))
 (segment (start 152.5905 51.8795) (end 156.21508 51.8795) (width 0.3048) (layer F.Cu) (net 4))
 (segment (start 151.003 53.467) (end 152.5905 51.8795) (width 0.3048) (layer F.Cu) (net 4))
 (segment (start 144.907 53.467) (end 151.003 53.467) (width 0.3048) (layer F.Cu) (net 4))
 (segment (start 142.367 50.927) (end 144.907 53.467) (width 0.3048) (layer F.Cu) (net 4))
 (segment (start 142.367 37.846) (end 142.367 50.927) (width 0.3048) (layer F.Cu) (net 4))
 (segment (start 142.494 37.719) (end 142.367 37.846) (width 0.3048) (layer F.Cu) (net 4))
 (via (at 142.494 37.719) (size 0.6) (drill 0.4) (layers F.Cu B.Cu) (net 4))
 (segment (start 142.5067 37.7063) (end 142.494 37.719) (width 0.3048) (layer B.Cu) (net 4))
 (segment (start 156.21508 50.6095) (end 152.8445 50.6095) (width 0.3048) (layer F.Cu) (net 5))
 (segment (start 144.6403 34.9377) (end 146.5326 34.9377) (width 0.3048) (layer F.Cu) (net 5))
 (segment (start 143.637 35.941) (end 144.6403 34.9377) (width 0.3048) (layer F.Cu) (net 5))
 (segment (start 143.637 49.53) (end 143.637 35.941) (width 0.3048) (layer F.Cu) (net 5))
 (segment (start 146.685 52.578) (end 143.637 49.53) (width 0.3048) (layer F.Cu) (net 5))
 (segment (start 150.876 52.578) (end 146.685 52.578) (width 0.3048) (layer F.Cu) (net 5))
 (segment (start 152.8445 50.6095) (end 150.876 52.578) (width 0.3048) (layer F.Cu) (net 5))
 (via (at 153.924 61.595) (size 0.6) (drill 0.4) (layers F.Cu B.Cu) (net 6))
 (segment (start 152.019 63.087) (end 153.702 63.087) (width 0.3048) (layer B.Cu) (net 6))
 (segment (start 153.924 62.865) (end 153.702 63.087) (width 0.3048) (layer B.Cu) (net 6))
 (segment (start 153.924 62.865) (end 153.924 61.595) (width 0.3048) (layer B.Cu) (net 6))
 (segment (start 141.605 61.595) (end 148.844 61.595) (width 0.3048) (layer F.Cu) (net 6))
 (segment (start 148.844 61.595) (end 153.924 61.595) (width 0.3048) (layer F.Cu) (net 6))
 (segment (start 153.924 61.595) (end 156.177 61.595) (width 0.3048) (layer F.Cu) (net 6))
 (segment (start 156.21 63.087) (end 156.21 62.23) (width 0.3048) (layer B.Cu) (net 7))
 (segment (start 156.21 62.23) (end 154.305 60.325) (width 0.3048) (layer B.Cu) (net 7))
 (segment (start 154.305 60.325) (end 154.051 60.325) (width 0.3048) (layer B.Cu) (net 7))
 (via (at 154.051 60.325) (size 0.6) (drill 0.4) (layers F.Cu B.Cu) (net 7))
 (segment (start 141.605 59.055) (end 149.225 59.055) (width 0.3048) (layer F.Cu) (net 7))
 (segment (start 150.495 60.325) (end 154.051 60.325) (width 0.3048) (layer F.Cu) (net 7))
 (segment (start 154.051 60.325) (end 156.177 60.325) (width 0.3048) (layer F.Cu) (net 7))
 (segment (start 149.225 59.055) (end 150.495 60.325) (width 0.3048) (layer F.Cu) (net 7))
 (segment (start 156.177 59.055) (end 154.178 59.055) (width 0.3048) (layer F.Cu) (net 8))
 (segment (start 154.178 59.055) (end 154.178 59.087) (width 0.3048) (layer B.Cu) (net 8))
 (via (at 154.178 59.055) (size 0.6) (drill 0.4) (layers F.Cu B.Cu) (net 8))
 (segment (start 156.21 59.087) (end 154.178 59.087) (width 0.3048) (layer B.Cu) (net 8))
 (segment (start 154.178 59.087) (end 152.019 59.087) (width 0.3048) (layer B.Cu) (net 8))
 (segment (start 161.577 62.865) (end 170.815 62.865) (width 0.3048) (layer F.Cu) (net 9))
 (segment (start 161.577 59.055) (end 168.275 59.055) (width 0.3048) (layer F.Cu) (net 11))
 (segment (start 169.545 60.325) (end 170.815 60.325) (width 0.3048) (layer F.Cu) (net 11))
 (segment (start 168.275 59.055) (end 169.545 60.325) (width 0.3048) (layer F.Cu) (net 11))
 (segment (start 161.41192 51.8795) (end 162.8775 51.8795) (width 0.3048) (layer F.Cu) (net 18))
 (segment (start 168.148 73.025) (end 170.815 73.025) (width 0.3048) (layer B.Cu) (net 18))
 (segment (start 165.227 70.104) (end 168.148 73.025) (width 0.3048) (layer B.Cu) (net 18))
 (segment (start 165.227 56.261) (end 165.227 70.104) (width 0.3048) (layer B.Cu) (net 18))
 (via (at 165.227 56.261) (size 0.6) (drill 0.4) (layers F.Cu B.Cu) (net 18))
 (segment (start 165.227 54.229) (end 165.227 56.261) (width 0.3048) (layer F.Cu) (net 18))
 (segment (start 162.8775 51.8795) (end 165.227 54.229) (width 0.3048) (layer F.Cu) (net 18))
 (segment (start 170.815 70.485) (end 168.656 70.485) (width 0.3048) (layer B.Cu) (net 19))
 (segment (start 163.1315 50.6095) (end 161.41192 50.6095) (width 0.3048) (layer F.Cu) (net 19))
 (segment (start 166.497 53.975) (end 163.1315 50.6095) (width 0.3048) (layer F.Cu) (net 19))
 (segment (start 166.497 56.261) (end 166.497 53.975) (width 0.3048) (layer F.Cu) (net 19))
 (via (at 166.497 56.261) (size 0.6) (drill 0.4) (layers F.Cu B.Cu) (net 19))
 (segment (start 166.497 68.326) (end 166.497 56.261) (width 0.3048) (layer B.Cu) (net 19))
 (segment (start 168.656 70.485) (end 166.497 68.326) (width 0.3048) (layer B.Cu) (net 19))
 (segment (start 161.41192 49.3395) (end 163.6395 49.3395) (width 0.3048) (layer F.Cu) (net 20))
 (segment (start 168.656 57.785) (end 170.815 57.785) (width 0.3048) (layer F.Cu) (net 20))
 (segment (start 167.513 56.642) (end 168.656 57.785) (width 0.3048) (layer F.Cu) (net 20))
 (segment (start 167.513 53.213) (end 167.513 56.642) (width 0.3048) (layer F.Cu) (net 20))
 (segment (start 163.6395 49.3395) (end 167.513 53.213) (width 0.3048) (layer F.Cu) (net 20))
 (segment (start 161.41192 48.0695) (end 164.1475 48.0695) (width 0.3048) (layer F.Cu) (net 21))
 (segment (start 169.164 55.245) (end 170.815 55.245) (width 0.3048) (layer F.Cu) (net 21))
 (segment (start 168.275 54.356) (end 169.164 55.245) (width 0.3048) (layer F.Cu) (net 21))
 (segment (start 168.275 52.197) (end 168.275 54.356) (width 0.3048) (layer F.Cu) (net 21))
 (segment (start 164.1475 48.0695) (end 168.275 52.197) (width 0.3048) (layer F.Cu) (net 21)))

